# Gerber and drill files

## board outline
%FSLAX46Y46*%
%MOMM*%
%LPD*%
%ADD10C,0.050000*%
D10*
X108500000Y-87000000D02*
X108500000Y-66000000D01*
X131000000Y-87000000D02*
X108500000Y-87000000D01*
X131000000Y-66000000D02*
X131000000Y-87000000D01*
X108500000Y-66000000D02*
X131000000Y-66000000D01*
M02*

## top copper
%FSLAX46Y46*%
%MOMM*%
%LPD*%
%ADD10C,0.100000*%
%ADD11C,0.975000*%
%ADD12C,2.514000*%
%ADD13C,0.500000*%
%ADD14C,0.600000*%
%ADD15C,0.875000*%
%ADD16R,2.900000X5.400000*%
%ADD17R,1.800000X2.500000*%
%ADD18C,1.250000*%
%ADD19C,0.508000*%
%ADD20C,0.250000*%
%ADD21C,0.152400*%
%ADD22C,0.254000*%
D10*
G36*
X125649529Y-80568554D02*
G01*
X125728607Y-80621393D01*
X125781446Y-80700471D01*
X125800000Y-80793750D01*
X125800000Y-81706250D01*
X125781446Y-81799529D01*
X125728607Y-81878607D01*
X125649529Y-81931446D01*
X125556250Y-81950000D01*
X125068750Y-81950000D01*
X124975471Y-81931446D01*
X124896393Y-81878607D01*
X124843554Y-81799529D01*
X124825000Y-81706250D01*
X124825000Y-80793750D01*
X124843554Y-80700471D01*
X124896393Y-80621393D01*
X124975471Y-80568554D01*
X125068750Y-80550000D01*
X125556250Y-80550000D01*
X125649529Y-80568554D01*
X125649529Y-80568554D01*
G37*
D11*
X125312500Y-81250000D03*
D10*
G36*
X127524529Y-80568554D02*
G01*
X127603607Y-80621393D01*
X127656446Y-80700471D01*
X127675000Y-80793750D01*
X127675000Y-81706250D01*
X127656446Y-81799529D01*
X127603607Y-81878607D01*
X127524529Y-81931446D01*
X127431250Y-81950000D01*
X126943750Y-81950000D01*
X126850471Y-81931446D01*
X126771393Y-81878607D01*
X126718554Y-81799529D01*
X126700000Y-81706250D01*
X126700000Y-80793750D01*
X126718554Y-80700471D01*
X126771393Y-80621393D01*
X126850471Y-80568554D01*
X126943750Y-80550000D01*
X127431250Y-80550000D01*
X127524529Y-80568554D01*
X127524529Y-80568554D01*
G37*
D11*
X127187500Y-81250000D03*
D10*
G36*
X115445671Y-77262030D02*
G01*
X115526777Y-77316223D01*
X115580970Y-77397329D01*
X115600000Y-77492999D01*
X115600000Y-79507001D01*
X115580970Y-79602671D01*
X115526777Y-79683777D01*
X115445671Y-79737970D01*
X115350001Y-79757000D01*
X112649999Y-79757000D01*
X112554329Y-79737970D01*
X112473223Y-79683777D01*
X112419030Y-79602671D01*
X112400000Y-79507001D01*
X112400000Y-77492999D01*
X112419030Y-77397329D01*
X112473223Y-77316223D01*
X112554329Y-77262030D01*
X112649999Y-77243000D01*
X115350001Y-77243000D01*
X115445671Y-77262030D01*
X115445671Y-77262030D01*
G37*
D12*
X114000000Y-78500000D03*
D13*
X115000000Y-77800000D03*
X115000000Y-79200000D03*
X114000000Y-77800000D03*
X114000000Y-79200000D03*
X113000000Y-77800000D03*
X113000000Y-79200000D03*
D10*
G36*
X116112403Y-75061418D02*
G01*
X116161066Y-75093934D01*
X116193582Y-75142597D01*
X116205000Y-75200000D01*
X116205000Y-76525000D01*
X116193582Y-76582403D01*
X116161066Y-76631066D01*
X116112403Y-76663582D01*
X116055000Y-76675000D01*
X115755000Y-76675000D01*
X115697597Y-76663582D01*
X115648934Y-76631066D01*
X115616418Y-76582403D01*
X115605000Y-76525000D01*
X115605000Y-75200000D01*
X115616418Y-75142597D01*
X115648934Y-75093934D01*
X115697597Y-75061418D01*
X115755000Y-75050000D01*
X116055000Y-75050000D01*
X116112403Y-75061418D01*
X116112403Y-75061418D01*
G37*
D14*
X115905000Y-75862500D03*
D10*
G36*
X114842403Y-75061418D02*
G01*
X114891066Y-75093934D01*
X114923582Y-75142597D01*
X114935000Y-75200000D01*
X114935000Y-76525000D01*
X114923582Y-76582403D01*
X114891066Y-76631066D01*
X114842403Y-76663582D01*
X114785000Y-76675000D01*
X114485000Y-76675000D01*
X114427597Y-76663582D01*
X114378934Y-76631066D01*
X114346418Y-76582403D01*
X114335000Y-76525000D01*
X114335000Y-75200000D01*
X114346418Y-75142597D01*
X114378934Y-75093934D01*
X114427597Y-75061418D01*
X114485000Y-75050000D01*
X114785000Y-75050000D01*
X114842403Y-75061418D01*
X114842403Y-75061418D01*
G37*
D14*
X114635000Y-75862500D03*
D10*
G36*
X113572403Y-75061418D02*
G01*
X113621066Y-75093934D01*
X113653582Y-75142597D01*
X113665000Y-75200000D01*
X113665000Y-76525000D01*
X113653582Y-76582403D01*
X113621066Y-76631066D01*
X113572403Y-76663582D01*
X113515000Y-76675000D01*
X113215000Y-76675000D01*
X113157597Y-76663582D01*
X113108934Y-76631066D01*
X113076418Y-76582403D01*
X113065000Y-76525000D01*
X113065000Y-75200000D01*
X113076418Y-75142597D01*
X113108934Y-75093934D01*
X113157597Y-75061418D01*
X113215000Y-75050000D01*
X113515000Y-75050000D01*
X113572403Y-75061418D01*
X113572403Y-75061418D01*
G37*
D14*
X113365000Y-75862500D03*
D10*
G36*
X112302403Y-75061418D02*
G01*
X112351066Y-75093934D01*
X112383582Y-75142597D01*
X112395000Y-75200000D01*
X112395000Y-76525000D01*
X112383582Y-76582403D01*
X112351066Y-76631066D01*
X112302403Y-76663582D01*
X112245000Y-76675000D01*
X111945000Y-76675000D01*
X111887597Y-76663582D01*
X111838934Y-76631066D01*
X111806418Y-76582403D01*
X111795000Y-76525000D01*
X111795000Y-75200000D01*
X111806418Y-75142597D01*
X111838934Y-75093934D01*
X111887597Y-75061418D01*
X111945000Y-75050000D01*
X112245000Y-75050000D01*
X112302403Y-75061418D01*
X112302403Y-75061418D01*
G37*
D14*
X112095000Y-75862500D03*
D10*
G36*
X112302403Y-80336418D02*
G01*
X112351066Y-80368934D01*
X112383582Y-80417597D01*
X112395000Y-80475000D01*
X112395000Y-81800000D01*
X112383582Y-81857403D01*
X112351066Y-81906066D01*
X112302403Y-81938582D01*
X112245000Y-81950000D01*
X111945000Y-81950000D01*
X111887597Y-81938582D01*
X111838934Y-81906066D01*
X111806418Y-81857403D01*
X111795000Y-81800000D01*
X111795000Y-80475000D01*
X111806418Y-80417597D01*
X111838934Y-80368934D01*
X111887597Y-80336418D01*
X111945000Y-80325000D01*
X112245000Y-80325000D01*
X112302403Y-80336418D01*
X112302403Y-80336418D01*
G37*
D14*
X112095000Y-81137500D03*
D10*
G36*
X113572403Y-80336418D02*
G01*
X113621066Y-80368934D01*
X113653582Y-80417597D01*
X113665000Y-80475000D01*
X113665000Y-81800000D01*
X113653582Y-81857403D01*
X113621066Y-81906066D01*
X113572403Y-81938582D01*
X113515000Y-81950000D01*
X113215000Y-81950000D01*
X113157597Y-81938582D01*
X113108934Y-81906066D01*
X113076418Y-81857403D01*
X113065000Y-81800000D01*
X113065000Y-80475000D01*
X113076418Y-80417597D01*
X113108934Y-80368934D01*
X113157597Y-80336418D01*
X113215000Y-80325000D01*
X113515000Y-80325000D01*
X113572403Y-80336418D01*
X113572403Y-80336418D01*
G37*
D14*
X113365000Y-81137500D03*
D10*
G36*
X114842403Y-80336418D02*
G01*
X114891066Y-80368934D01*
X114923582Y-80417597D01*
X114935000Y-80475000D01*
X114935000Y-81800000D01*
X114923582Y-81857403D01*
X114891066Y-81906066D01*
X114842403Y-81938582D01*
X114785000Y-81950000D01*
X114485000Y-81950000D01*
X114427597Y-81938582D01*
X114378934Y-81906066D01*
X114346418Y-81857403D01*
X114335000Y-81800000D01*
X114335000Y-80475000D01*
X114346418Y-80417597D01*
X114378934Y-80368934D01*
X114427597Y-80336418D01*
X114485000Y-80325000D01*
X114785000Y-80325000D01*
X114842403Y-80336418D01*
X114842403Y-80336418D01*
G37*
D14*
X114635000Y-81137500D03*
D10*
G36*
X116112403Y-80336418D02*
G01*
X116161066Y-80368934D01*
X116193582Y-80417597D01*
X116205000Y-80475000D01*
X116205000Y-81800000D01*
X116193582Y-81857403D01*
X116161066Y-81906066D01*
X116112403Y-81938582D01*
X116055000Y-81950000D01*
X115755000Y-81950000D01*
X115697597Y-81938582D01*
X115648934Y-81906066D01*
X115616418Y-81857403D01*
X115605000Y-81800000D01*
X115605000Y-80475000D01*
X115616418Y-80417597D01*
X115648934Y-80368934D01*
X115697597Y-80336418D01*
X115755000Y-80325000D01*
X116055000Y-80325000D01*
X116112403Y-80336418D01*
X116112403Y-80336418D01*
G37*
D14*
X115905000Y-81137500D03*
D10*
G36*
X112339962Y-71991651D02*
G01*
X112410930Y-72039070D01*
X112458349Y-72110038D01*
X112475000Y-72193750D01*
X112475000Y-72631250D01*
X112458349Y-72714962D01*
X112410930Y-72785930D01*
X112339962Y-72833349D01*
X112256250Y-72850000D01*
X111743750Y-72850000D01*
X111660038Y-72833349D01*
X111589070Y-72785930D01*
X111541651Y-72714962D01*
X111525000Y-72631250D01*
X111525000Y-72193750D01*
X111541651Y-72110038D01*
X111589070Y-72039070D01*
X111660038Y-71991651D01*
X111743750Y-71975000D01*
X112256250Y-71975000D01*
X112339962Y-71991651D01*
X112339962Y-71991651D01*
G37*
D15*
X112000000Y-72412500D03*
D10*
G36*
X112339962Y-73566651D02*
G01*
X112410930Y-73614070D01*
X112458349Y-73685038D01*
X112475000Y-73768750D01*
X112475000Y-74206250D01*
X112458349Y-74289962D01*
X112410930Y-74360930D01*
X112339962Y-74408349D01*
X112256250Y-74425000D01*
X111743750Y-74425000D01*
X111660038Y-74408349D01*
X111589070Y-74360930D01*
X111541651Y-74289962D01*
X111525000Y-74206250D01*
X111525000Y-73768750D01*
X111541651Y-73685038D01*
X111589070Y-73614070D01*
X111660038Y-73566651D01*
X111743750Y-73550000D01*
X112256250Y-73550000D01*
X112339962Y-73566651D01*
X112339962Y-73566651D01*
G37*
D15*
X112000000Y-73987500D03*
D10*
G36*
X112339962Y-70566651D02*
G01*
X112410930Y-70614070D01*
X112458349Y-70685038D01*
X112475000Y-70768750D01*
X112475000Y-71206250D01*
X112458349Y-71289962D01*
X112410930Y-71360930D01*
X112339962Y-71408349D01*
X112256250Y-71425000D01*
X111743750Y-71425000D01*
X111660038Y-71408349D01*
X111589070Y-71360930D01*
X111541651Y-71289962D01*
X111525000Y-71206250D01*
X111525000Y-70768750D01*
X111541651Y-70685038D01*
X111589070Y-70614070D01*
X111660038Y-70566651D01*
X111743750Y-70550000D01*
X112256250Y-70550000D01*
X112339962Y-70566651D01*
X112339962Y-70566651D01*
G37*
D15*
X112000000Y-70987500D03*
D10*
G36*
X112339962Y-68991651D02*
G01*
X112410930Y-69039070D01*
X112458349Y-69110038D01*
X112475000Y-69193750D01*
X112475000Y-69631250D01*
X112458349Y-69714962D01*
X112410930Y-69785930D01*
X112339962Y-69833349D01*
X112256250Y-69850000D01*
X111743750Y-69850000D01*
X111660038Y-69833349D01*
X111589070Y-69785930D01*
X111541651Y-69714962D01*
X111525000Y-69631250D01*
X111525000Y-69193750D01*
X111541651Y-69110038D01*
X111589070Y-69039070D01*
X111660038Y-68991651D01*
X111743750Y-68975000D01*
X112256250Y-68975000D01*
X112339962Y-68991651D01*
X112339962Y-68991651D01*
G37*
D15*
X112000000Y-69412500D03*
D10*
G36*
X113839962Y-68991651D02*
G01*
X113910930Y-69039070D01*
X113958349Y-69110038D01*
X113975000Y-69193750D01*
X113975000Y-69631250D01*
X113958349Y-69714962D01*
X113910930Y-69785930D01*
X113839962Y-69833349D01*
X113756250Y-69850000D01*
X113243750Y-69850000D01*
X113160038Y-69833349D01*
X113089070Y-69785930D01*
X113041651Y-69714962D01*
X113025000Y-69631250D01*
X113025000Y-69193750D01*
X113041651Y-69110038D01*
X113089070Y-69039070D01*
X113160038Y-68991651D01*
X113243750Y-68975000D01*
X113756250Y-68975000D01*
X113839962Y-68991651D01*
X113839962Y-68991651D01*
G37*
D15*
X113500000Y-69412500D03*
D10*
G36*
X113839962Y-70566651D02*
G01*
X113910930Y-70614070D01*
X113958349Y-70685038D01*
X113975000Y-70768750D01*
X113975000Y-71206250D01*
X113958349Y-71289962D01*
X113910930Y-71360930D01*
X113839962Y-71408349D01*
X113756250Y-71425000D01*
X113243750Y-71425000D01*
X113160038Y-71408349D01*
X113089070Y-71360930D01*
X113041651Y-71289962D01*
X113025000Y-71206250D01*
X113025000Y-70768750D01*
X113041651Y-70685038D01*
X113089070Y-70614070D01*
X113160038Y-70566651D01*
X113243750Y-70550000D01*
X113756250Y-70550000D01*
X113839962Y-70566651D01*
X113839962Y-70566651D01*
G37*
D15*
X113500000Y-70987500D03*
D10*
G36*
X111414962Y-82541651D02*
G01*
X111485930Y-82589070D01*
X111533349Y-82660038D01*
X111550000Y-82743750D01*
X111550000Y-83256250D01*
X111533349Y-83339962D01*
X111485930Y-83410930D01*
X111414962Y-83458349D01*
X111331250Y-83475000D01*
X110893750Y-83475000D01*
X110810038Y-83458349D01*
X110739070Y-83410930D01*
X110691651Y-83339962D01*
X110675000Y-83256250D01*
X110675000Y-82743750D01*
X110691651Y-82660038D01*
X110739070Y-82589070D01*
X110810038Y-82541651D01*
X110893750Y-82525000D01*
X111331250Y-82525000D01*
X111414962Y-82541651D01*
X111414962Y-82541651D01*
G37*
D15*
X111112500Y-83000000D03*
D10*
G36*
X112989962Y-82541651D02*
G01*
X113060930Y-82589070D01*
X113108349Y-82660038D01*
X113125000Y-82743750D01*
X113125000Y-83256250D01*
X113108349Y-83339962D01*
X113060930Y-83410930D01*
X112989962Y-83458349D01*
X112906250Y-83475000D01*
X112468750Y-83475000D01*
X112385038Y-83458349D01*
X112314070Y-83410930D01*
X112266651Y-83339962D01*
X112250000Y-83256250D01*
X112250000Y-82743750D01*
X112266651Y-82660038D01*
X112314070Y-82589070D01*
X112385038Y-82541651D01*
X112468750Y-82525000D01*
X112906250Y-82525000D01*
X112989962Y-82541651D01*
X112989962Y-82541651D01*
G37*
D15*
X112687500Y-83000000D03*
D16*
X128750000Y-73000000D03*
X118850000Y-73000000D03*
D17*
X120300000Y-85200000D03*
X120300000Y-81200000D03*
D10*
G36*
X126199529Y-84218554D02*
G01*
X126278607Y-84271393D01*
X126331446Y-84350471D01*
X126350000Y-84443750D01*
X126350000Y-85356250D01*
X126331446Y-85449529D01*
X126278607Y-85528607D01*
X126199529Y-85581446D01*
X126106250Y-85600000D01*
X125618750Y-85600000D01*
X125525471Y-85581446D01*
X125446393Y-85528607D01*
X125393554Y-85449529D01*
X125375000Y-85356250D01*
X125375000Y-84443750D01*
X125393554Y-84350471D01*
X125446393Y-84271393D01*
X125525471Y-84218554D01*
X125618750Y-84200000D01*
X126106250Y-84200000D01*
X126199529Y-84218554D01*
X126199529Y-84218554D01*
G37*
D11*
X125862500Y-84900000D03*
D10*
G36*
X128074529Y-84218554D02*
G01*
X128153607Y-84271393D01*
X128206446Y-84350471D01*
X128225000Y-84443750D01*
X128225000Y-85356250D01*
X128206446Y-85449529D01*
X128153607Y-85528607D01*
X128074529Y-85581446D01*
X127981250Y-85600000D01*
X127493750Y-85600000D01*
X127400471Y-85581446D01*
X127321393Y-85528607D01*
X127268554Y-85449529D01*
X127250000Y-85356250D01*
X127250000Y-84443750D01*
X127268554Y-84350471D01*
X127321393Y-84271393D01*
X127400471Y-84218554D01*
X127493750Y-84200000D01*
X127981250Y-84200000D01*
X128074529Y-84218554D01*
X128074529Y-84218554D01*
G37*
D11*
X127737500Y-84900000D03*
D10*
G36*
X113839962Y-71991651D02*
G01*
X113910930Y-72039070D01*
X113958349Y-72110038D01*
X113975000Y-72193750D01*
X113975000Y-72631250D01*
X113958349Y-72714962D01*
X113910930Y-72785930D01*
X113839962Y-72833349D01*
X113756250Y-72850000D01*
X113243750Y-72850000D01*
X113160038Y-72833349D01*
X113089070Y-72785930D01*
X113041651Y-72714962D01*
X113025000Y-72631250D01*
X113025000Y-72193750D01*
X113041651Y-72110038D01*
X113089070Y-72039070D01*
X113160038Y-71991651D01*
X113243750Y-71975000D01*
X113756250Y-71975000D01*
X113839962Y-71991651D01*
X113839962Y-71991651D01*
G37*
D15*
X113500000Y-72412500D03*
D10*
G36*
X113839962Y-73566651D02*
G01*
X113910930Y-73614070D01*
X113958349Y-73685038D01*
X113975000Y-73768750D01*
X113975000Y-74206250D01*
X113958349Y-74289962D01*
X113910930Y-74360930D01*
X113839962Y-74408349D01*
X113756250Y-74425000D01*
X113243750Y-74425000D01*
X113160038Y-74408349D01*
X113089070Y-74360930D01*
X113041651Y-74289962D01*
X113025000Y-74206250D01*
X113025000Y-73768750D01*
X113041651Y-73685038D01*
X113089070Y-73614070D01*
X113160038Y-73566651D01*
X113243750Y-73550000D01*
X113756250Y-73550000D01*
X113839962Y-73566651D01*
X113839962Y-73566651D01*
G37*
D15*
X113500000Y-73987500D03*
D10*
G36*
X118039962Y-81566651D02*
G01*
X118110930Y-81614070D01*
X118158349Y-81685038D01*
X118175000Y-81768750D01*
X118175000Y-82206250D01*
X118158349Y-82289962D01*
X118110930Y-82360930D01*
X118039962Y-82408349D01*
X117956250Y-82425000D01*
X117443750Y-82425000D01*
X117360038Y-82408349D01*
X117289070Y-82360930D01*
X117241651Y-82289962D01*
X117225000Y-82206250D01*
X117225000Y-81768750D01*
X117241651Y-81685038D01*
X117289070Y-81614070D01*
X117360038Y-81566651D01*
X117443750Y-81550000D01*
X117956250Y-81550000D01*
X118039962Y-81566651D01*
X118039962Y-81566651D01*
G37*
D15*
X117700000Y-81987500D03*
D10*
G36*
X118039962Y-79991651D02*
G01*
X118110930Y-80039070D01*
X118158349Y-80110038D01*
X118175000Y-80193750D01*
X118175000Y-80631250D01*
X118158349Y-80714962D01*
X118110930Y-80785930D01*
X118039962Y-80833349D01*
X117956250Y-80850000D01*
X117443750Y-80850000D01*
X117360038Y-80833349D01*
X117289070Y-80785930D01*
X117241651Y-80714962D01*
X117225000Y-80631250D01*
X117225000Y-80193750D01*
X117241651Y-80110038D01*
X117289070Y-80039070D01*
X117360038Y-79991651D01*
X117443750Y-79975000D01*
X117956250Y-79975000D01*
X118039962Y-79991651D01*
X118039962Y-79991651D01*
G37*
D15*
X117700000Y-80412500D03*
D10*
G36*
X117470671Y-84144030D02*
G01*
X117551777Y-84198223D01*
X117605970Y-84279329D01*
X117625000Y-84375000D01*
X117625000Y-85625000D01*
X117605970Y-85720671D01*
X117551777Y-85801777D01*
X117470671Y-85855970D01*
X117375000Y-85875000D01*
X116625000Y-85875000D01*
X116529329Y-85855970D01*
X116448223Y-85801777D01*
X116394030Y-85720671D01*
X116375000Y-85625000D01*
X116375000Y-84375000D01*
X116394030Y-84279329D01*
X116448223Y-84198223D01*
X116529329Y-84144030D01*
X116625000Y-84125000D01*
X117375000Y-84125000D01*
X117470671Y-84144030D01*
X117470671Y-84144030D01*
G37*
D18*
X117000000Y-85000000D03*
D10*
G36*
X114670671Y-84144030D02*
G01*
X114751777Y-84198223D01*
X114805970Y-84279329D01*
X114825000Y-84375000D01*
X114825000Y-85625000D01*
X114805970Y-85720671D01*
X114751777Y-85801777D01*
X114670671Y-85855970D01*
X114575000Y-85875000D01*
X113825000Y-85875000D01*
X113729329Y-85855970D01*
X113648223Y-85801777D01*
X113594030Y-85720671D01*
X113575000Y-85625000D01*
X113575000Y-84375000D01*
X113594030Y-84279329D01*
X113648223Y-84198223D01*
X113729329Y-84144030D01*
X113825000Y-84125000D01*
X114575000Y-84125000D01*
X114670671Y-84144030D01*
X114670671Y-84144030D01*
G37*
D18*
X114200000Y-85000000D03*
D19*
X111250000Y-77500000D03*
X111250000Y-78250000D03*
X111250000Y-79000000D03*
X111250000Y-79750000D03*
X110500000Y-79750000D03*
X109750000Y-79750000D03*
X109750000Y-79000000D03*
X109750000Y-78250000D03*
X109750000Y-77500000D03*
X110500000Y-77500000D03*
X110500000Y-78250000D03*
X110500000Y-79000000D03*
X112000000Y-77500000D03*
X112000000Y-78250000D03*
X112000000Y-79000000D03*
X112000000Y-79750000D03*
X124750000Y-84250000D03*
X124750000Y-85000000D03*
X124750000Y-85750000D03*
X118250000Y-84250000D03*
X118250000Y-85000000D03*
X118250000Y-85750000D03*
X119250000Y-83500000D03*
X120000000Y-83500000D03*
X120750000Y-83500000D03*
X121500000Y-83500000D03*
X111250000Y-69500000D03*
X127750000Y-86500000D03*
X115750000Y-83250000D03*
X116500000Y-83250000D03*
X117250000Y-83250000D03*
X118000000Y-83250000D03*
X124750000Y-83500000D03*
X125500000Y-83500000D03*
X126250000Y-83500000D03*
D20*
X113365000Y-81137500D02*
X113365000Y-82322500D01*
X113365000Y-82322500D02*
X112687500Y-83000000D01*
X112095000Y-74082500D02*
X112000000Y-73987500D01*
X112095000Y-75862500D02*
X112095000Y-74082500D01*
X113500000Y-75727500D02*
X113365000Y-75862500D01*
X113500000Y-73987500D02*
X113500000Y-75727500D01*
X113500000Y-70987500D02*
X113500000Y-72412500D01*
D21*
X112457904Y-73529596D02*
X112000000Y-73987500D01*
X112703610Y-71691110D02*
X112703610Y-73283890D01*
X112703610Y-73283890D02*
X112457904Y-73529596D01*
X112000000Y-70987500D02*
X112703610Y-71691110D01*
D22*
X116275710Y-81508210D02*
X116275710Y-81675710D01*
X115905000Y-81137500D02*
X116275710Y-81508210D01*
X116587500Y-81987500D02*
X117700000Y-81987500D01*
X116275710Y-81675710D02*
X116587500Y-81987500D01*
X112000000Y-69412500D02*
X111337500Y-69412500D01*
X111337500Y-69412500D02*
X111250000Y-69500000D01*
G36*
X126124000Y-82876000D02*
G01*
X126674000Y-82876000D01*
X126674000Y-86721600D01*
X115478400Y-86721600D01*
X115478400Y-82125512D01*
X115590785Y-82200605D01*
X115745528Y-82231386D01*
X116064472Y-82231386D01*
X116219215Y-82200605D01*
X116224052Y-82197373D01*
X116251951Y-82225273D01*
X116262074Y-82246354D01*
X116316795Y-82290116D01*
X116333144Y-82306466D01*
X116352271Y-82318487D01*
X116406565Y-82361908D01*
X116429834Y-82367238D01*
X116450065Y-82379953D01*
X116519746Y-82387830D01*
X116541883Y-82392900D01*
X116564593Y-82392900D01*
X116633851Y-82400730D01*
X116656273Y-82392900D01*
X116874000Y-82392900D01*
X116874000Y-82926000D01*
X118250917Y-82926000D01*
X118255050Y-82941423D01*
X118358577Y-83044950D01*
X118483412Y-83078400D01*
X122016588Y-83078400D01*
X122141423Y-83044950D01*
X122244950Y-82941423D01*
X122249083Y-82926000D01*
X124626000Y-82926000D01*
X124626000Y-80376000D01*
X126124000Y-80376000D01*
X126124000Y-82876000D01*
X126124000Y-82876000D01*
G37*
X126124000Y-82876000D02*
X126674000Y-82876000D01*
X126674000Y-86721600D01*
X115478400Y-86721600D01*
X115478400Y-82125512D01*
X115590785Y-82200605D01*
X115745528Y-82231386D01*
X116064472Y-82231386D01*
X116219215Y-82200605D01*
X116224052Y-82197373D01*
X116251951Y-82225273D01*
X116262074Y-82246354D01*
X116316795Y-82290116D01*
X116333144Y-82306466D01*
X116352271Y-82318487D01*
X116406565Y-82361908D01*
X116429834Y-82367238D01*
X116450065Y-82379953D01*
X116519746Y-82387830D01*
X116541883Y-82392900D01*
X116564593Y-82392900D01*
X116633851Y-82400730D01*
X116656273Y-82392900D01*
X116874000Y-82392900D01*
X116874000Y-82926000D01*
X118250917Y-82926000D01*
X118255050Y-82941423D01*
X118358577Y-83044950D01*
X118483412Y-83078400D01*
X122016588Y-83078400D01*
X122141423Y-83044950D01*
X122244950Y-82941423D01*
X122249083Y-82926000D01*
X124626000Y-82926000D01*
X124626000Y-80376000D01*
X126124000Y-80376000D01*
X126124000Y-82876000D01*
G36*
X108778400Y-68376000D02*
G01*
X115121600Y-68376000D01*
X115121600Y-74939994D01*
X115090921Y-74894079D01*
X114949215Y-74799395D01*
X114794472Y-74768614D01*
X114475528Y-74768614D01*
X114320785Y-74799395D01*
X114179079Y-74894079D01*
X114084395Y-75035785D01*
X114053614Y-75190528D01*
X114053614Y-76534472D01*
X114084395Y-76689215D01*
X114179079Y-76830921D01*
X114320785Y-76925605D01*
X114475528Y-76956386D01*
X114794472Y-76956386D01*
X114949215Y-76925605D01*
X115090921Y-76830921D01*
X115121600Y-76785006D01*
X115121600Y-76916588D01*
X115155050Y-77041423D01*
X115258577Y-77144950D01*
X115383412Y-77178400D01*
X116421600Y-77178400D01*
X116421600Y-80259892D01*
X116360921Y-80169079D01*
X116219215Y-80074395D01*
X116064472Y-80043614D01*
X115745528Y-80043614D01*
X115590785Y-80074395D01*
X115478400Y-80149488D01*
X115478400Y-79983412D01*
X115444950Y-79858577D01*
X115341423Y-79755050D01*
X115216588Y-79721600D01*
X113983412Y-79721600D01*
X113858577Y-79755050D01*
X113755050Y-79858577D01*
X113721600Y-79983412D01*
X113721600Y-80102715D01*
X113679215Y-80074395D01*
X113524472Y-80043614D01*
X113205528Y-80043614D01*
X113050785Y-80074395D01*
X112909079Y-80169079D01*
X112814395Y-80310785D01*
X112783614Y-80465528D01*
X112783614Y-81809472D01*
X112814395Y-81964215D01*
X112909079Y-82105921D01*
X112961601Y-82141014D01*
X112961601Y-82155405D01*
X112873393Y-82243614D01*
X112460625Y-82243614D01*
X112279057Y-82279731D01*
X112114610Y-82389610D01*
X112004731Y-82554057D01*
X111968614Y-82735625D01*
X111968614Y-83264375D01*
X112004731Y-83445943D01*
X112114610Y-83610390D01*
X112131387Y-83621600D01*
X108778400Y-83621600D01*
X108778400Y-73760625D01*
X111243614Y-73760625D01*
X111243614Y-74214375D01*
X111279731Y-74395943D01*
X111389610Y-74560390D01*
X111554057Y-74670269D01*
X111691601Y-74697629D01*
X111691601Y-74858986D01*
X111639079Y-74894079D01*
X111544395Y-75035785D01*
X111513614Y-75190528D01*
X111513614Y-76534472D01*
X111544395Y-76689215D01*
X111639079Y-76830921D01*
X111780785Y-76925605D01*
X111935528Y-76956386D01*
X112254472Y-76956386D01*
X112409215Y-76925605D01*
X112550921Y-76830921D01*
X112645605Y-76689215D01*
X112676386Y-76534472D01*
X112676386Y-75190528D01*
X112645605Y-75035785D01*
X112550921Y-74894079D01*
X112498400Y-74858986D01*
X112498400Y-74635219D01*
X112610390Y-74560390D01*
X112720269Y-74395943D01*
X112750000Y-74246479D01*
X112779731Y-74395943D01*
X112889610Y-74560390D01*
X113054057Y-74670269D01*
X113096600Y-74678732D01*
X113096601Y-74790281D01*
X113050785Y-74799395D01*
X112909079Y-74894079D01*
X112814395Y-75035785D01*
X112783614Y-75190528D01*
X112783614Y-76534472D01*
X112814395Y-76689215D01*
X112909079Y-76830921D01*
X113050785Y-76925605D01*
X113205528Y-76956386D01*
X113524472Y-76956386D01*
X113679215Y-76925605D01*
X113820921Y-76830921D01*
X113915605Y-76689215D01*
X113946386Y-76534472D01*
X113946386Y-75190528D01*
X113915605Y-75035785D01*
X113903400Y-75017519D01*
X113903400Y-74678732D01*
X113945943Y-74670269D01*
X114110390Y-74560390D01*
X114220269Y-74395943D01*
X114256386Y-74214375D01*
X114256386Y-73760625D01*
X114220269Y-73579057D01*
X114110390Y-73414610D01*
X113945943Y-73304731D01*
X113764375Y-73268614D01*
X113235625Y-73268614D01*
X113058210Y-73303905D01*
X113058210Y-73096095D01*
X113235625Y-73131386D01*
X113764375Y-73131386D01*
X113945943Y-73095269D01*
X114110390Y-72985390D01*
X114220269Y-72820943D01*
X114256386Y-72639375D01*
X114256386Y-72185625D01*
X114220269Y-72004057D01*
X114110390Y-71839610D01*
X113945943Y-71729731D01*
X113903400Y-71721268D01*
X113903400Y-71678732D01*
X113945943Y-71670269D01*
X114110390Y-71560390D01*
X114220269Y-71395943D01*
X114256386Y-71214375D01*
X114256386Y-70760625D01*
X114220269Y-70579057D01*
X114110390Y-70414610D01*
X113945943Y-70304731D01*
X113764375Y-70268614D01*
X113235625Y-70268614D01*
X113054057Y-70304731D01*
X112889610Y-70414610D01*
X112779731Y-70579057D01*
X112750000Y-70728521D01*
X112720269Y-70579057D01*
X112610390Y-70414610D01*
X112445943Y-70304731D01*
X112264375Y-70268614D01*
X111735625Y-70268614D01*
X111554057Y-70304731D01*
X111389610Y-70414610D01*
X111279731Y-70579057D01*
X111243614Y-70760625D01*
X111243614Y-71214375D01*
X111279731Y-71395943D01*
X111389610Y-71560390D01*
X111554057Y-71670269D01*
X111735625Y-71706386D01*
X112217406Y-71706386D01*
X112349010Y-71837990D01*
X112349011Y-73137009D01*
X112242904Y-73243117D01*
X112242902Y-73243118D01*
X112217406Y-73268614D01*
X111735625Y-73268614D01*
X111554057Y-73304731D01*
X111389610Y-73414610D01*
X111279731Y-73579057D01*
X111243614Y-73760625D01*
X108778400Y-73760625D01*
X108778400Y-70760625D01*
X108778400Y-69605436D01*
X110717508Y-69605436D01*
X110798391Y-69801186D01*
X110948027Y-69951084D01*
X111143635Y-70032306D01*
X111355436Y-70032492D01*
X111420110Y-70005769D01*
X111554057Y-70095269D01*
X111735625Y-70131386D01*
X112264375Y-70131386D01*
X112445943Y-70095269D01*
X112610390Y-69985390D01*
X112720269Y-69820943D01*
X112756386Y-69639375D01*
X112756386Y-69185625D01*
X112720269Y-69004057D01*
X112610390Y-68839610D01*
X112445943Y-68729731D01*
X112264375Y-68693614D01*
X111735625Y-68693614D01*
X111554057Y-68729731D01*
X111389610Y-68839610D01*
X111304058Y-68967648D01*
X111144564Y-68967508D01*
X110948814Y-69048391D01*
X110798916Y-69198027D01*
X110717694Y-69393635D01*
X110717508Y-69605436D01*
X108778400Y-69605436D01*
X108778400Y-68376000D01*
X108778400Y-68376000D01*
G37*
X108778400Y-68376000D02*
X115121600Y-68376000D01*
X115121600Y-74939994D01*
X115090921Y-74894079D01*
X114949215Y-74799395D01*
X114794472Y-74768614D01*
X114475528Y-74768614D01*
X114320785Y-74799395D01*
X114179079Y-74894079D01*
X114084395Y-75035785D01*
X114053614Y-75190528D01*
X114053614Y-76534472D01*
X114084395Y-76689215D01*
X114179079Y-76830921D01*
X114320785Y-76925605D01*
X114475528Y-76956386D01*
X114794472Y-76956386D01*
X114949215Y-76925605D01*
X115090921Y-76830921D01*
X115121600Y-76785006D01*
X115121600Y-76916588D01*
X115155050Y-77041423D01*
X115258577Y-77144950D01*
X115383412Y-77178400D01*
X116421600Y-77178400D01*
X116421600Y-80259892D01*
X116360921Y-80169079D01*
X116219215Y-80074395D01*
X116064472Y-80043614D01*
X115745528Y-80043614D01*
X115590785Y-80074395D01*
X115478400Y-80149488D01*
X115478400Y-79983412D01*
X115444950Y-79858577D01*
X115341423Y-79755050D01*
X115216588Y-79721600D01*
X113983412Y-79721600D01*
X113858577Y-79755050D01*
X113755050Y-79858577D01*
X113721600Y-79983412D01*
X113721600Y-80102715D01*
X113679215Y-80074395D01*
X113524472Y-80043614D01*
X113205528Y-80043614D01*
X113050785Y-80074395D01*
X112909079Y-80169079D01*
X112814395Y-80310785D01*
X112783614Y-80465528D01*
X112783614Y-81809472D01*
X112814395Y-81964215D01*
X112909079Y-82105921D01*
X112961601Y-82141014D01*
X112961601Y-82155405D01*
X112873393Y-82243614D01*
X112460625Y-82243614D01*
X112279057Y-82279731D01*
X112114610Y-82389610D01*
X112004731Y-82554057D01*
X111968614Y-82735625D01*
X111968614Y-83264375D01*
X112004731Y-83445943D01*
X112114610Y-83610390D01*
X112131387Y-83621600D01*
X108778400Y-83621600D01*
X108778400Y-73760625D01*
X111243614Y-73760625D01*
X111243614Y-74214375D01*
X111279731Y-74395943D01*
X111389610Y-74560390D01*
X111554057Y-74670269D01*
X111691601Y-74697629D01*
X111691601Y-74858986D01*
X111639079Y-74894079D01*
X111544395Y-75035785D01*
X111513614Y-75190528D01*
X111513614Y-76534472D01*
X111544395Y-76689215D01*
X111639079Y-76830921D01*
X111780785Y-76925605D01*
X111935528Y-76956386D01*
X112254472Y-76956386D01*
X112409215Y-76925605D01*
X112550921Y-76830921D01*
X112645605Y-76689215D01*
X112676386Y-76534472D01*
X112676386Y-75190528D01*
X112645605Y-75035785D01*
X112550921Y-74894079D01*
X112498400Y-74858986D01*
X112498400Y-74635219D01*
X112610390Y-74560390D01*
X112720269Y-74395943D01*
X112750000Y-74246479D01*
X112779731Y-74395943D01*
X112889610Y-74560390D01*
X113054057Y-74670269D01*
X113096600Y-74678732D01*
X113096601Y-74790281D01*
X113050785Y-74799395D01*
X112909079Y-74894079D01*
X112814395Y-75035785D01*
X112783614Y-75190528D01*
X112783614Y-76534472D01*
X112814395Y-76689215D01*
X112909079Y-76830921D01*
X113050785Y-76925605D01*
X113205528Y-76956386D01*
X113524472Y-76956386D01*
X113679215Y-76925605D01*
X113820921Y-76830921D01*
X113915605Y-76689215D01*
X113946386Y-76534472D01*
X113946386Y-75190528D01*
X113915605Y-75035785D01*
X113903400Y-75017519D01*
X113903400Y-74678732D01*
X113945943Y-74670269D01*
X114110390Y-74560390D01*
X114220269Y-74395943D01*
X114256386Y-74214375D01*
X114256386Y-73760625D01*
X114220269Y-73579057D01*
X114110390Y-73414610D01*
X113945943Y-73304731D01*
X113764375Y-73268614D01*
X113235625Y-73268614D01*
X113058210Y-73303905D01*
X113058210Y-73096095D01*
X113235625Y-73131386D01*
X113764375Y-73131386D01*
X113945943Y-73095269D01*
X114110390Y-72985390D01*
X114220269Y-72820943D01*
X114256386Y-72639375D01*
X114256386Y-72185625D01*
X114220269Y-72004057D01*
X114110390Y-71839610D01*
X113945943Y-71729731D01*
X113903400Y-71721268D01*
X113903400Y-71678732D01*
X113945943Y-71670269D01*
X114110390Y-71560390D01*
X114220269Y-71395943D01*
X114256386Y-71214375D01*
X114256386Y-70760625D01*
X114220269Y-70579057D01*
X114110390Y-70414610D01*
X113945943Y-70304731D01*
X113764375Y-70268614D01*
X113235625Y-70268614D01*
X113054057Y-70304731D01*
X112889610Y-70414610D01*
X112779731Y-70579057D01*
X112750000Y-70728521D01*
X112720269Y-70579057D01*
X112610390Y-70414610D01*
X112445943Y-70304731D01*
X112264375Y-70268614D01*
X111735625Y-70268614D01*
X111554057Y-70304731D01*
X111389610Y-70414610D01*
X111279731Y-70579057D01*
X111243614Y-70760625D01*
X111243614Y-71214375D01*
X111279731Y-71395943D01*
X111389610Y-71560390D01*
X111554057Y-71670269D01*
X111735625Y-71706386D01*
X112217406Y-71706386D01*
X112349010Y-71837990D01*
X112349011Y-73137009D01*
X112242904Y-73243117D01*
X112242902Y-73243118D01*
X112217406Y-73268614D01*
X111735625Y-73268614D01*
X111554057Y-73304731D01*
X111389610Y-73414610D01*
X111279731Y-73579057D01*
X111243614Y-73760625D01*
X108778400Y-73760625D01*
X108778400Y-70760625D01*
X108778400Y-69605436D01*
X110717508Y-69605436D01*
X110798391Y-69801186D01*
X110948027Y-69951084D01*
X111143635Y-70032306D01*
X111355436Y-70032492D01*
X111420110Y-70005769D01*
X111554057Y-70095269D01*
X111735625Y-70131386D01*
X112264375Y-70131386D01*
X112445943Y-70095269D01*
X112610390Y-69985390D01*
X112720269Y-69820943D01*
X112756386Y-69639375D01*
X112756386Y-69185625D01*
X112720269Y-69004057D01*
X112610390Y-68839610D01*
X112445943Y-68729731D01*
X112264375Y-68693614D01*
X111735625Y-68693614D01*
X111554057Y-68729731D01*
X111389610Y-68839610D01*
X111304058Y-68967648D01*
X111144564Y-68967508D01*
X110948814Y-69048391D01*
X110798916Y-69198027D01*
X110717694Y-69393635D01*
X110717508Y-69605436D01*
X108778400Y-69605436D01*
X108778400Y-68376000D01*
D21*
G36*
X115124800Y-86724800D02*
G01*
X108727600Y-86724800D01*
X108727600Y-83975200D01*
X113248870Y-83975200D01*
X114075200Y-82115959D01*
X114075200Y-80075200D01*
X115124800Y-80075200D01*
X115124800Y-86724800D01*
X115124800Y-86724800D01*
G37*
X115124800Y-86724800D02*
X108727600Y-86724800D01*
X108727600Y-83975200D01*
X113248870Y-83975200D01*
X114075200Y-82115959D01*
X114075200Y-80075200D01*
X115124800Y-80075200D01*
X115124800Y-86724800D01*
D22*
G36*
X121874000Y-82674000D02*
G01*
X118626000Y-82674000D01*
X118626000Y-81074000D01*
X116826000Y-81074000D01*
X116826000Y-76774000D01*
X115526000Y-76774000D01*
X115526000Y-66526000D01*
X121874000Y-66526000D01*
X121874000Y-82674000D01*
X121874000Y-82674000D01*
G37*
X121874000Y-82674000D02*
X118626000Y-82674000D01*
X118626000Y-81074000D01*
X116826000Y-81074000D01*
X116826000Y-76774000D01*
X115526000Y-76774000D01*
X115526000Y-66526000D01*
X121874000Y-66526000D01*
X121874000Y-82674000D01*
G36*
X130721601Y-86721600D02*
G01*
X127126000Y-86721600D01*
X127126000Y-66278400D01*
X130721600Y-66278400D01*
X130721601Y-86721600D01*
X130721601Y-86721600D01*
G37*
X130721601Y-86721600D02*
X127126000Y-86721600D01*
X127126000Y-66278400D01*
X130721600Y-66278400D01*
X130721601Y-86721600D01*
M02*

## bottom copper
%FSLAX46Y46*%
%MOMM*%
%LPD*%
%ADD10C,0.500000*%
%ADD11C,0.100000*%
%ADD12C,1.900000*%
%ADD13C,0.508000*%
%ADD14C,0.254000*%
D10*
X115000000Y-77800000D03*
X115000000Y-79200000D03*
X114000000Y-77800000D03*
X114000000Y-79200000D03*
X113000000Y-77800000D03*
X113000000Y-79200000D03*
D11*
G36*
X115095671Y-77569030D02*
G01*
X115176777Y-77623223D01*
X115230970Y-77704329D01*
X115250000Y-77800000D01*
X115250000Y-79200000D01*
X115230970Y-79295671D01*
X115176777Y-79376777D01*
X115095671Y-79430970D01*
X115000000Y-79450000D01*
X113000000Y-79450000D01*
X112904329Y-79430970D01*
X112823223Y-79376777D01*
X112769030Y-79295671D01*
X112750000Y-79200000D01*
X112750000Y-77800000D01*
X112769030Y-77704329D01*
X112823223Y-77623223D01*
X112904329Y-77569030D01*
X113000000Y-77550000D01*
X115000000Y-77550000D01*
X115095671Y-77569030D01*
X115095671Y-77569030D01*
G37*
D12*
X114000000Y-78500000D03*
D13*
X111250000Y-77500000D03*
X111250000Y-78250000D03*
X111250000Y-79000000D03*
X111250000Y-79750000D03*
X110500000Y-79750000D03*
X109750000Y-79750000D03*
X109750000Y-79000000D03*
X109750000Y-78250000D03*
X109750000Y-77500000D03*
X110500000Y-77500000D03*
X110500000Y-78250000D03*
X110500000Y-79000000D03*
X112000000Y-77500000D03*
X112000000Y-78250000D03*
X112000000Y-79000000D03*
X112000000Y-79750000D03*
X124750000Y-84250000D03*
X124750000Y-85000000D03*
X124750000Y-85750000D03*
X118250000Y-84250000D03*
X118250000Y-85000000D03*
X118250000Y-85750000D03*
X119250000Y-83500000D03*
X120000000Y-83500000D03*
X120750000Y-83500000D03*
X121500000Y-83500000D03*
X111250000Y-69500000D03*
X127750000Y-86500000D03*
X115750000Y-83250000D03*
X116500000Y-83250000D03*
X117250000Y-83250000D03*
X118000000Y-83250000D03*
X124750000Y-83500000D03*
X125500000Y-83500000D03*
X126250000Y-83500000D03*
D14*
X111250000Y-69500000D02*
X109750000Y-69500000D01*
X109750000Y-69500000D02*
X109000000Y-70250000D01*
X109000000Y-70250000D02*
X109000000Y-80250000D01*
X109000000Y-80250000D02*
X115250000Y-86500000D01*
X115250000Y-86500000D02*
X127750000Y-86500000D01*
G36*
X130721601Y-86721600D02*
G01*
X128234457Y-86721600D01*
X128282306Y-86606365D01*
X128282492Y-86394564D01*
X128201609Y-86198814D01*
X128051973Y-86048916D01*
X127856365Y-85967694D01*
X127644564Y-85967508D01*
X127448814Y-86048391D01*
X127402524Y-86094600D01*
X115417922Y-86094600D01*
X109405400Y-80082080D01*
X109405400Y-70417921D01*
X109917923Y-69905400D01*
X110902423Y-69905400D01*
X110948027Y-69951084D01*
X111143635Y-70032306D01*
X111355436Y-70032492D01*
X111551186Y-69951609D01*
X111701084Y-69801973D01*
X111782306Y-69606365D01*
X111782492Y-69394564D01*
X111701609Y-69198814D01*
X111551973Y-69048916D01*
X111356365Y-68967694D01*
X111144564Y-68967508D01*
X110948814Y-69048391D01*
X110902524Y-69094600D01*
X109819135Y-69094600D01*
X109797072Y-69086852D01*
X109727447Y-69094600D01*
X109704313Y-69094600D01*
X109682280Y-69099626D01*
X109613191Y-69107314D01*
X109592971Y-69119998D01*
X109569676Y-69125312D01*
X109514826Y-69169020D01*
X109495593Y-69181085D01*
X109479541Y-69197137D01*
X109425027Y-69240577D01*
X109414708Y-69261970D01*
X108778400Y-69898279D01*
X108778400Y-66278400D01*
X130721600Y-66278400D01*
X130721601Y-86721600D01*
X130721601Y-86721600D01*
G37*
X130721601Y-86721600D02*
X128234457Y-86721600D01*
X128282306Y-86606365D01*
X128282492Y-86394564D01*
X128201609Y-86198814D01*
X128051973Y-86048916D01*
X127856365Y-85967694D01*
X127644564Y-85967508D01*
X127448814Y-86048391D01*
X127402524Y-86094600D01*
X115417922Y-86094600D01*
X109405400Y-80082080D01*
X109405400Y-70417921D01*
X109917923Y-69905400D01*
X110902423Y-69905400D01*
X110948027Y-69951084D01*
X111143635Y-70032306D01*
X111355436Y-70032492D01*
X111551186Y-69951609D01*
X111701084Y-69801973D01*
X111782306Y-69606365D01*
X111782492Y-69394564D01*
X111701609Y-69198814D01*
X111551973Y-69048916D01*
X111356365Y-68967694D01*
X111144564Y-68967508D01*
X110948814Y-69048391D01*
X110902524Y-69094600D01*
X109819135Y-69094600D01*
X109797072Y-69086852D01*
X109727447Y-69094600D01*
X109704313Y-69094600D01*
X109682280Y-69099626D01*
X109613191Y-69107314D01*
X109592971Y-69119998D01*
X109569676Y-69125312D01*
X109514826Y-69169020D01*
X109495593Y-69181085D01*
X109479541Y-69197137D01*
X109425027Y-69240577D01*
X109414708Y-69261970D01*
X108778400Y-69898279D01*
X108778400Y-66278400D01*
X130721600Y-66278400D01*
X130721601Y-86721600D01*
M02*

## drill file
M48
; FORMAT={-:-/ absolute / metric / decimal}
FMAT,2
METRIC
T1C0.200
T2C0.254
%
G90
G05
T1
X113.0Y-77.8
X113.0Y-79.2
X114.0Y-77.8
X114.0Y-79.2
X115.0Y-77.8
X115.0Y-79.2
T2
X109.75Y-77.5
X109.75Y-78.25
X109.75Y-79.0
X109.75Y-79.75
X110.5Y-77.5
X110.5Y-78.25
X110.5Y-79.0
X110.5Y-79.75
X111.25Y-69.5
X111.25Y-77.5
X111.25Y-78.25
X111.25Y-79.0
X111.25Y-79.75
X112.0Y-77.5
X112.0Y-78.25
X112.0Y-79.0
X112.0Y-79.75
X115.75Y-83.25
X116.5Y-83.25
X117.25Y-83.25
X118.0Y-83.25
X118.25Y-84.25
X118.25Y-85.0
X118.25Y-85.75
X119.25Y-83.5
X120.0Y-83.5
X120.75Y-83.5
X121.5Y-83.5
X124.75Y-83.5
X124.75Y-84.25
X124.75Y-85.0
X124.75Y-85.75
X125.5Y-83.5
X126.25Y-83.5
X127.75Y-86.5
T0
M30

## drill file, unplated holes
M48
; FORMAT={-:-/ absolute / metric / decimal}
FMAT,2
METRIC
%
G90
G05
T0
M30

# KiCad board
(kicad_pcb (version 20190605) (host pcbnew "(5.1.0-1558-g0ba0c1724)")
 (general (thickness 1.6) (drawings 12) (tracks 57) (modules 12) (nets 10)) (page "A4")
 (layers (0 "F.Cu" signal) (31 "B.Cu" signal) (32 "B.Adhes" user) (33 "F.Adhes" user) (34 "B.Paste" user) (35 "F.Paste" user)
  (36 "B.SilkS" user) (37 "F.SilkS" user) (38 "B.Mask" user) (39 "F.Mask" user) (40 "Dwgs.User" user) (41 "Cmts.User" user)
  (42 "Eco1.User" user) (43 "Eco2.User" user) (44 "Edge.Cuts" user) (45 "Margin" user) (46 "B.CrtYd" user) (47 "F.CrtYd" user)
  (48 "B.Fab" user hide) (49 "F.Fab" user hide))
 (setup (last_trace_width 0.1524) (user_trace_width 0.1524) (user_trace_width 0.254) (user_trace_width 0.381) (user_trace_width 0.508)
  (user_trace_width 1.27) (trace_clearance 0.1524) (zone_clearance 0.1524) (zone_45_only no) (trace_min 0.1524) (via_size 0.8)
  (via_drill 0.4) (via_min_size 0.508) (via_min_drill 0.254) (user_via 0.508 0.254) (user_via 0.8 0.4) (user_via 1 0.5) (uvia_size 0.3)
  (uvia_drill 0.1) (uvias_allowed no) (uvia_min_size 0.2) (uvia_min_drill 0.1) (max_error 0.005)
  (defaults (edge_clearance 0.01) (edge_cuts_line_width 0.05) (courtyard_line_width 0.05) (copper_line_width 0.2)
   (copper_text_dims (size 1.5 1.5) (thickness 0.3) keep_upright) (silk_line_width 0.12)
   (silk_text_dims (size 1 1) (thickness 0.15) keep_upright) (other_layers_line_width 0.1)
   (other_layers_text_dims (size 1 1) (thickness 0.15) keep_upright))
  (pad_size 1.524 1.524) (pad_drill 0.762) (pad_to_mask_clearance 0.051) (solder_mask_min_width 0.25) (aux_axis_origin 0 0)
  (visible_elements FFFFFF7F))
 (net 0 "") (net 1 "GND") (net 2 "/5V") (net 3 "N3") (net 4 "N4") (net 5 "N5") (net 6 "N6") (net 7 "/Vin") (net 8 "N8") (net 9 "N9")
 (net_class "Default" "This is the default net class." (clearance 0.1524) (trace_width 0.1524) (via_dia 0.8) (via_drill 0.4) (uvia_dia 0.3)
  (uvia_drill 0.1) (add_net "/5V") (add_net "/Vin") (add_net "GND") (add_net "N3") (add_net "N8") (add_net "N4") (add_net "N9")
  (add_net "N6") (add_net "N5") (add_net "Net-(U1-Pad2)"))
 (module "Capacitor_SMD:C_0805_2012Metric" (layer "F.Cu") (at 126.25 81.25 180)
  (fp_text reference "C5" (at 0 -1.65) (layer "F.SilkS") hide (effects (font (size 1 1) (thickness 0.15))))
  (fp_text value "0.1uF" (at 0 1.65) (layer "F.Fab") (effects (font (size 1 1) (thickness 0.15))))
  (pad "2" smd roundrect (at 0.9375 0 180) (size 0.975 1.4) (layers "F.Cu" "F.Paste" "F.Mask") (roundrect_rratio 0.25) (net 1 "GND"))
  (pad "1" smd roundrect (at -0.9375 0 180) (size 0.975 1.4) (layers "F.Cu" "F.Paste" "F.Mask") (roundrect_rratio 0.25) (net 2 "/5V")))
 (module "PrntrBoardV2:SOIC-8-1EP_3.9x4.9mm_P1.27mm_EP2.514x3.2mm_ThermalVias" (layer "F.Cu") (at 114 78.5 270)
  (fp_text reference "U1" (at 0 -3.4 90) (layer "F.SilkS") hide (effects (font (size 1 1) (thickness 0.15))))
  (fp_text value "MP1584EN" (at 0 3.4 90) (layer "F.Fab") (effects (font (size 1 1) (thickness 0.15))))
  (pad "9" smd roundrect (at 0 0 270) (size 2.514 3.2) (layers "F.Cu" "F.Mask") (roundrect_rratio 0.099443) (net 1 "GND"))
  (pad "9" thru_hole circle (at -0.7 -1 270) (size 0.5 0.5) (drill 0.2) (layers *.Cu) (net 1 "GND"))
  (pad "9" thru_hole circle (at 0.7 -1 270) (size 0.5 0.5) (drill 0.2) (layers *.Cu) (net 1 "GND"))
  (pad "9" thru_hole circle (at -0.7 0 270) (size 0.5 0.5) (drill 0.2) (layers *.Cu) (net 1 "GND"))
  (pad "9" thru_hole circle (at 0.7 0 270) (size 0.5 0.5) (drill 0.2) (layers *.Cu) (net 1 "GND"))
  (pad "9" thru_hole circle (at -0.7 1 270) (size 0.5 0.5) (drill 0.2) (layers *.Cu) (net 1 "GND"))
  (pad "9" thru_hole circle (at 0.7 1 270) (size 0.5 0.5) (drill 0.2) (layers *.Cu) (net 1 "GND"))
  (pad "9" smd roundrect (at 0 0 270) (size 1.9 2.5) (layers "B.Cu") (roundrect_rratio 0.131579) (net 1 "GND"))
  (pad "" smd roundrect (at -0.63 -0.8 270) (size 1.05 1.34) (layers "F.Paste") (roundrect_rratio 0.238095))
  (pad "" smd roundrect (at -0.63 0.8 270) (size 1.05 1.34) (layers "F.Paste") (roundrect_rratio 0.238095))
  (pad "" smd roundrect (at 0.63 -0.8 270) (size 1.05 1.34) (layers "F.Paste") (roundrect_rratio 0.238095))
  (pad "" smd roundrect (at 0.63 0.8 270) (size 1.05 1.34) (layers "F.Paste") (roundrect_rratio 0.238095))
  (pad "1" smd roundrect (at -2.6375 -1.905 270) (size 1.625 0.6) (layers "F.Cu" "F.Paste" "F.Mask") (roundrect_rratio 0.25) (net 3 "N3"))
  (pad "2" smd roundrect (at -2.6375 -0.635 270) (size 1.625 0.6) (layers "F.Cu" "F.Paste" "F.Mask") (roundrect_rratio 0.25))
  (pad "3" smd roundrect (at -2.6375 0.635 270) (size 1.625 0.6) (layers "F.Cu" "F.Paste" "F.Mask") (roundrect_rratio 0.25) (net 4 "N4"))
  (pad "4" smd roundrect (at -2.6375 1.905 270) (size 1.625 0.6) (layers "F.Cu" "F.Paste" "F.Mask") (roundrect_rratio 0.25) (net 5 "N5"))
  (pad "5" smd roundrect (at 2.6375 1.905 270) (size 1.625 0.6) (layers "F.Cu" "F.Paste" "F.Mask") (roundrect_rratio 0.25) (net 1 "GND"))
  (pad "6" smd roundrect (at 2.6375 0.635 270) (size 1.625 0.6) (layers "F.Cu" "F.Paste" "F.Mask") (roundrect_rratio 0.25) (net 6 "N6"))
  (pad "7" smd roundrect (at 2.6375 -0.635 270) (size 1.625 0.6) (layers "F.Cu" "F.Paste" "F.Mask") (roundrect_rratio 0.25) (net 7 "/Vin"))
  (pad "8" smd roundrect (at 2.6375 -1.905 270) (size 1.625 0.6) (layers "F.Cu" "F.Paste" "F.Mask") (roundrect_rratio 0.25) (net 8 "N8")))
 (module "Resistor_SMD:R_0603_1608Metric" (layer "F.Cu") (at 112 73.2 90)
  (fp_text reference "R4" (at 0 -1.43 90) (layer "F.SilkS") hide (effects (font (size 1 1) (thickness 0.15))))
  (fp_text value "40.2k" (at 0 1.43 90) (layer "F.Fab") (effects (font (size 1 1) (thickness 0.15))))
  (pad "2" smd roundrect (at 0.7875 0 90) (size 0.875 0.95) (layers "F.Cu" "F.Paste" "F.Mask") (roundrect_rratio 0.25) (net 1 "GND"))
  (pad "1" smd roundrect (at -0.7875 0 90) (size 0.875 0.95) (layers "F.Cu" "F.Paste" "F.Mask") (roundrect_rratio 0.25) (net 5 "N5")))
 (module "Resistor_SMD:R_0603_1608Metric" (layer "F.Cu") (at 112 70.2 270)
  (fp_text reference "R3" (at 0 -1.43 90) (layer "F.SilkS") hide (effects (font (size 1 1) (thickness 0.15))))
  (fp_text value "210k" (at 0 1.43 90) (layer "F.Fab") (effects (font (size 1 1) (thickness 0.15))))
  (pad "2" smd roundrect (at 0.7875 0 270) (size 0.875 0.95) (layers "F.Cu" "F.Paste" "F.Mask") (roundrect_rratio 0.25) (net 5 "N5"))
  (pad "1" smd roundrect (at -0.7875 0 270) (size 0.875 0.95) (layers "F.Cu" "F.Paste" "F.Mask") (roundrect_rratio 0.25) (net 2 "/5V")))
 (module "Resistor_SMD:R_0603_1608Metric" (layer "F.Cu") (at 113.5 70.2 90)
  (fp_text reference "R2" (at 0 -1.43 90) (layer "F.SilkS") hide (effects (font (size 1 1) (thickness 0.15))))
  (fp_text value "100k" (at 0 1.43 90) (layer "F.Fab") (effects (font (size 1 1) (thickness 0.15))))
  (pad "2" smd roundrect (at 0.7875 0 90) (size 0.875 0.95) (layers "F.Cu" "F.Paste" "F.Mask") (roundrect_rratio 0.25) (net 1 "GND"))
  (pad "1" smd roundrect (at -0.7875 0 90) (size 0.875 0.95) (layers "F.Cu" "F.Paste" "F.Mask") (roundrect_rratio 0.25) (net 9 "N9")))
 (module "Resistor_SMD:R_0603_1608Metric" (layer "F.Cu") (at 111.9 83 180)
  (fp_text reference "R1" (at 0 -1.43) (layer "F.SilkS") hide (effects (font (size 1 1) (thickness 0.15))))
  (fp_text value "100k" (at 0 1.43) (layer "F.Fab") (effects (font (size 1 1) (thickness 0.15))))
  (pad "2" smd roundrect (at 0.7875 0 180) (size 0.875 0.95) (layers "F.Cu" "F.Paste" "F.Mask") (roundrect_rratio 0.25) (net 1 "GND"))
  (pad "1" smd roundrect (at -0.7875 0 180) (size 0.875 0.95) (layers "F.Cu" "F.Paste" "F.Mask") (roundrect_rratio 0.25) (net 6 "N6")))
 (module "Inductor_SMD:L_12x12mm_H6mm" (layer "F.Cu") (at 123.8 73)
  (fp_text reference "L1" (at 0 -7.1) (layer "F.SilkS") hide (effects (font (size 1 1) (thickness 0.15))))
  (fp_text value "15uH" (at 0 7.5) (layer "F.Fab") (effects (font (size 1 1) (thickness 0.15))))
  (pad "2" smd rect (at 4.95 0) (size 2.9 5.4) (layers "F.Cu" "F.Paste" "F.Mask") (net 2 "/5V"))
  (pad "1" smd rect (at -4.95 0) (size 2.9 5.4) (layers "F.Cu" "F.Paste" "F.Mask") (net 3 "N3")))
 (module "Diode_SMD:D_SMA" (layer "F.Cu") (at 120.3 83.2 270)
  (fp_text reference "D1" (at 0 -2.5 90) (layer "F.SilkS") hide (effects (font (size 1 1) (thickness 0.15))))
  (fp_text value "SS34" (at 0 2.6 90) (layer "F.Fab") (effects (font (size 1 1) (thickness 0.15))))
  (pad "2" smd rect (at 2 0 270) (size 2.5 1.8) (layers "F.Cu" "F.Paste" "F.Mask") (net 1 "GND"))
  (pad "1" smd rect (at -2 0 270) (size 2.5 1.8) (layers "F.Cu" "F.Paste" "F.Mask") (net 3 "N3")))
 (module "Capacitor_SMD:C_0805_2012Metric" (layer "F.Cu") (at 126.8 84.9 180)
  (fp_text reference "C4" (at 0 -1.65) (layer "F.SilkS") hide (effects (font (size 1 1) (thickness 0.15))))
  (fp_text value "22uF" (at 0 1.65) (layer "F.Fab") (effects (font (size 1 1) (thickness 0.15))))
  (pad "2" smd roundrect (at 0.9375 0 180) (size 0.975 1.4) (layers "F.Cu" "F.Paste" "F.Mask") (roundrect_rratio 0.25) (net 1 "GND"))
  (pad "1" smd roundrect (at -0.9375 0 180) (size 0.975 1.4) (layers "F.Cu" "F.Paste" "F.Mask") (roundrect_rratio 0.25) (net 2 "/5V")))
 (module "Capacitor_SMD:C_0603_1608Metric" (layer "F.Cu") (at 113.5 73.2 90)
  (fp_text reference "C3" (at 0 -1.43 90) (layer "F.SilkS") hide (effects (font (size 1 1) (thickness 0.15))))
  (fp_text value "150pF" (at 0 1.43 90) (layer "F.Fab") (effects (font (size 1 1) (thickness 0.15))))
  (pad "2" smd roundrect (at 0.7875 0 90) (size 0.875 0.95) (layers "F.Cu" "F.Paste" "F.Mask") (roundrect_rratio 0.25) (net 9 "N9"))
  (pad "1" smd roundrect (at -0.7875 0 90) (size 0.875 0.95) (layers "F.Cu" "F.Paste" "F.Mask") (roundrect_rratio 0.25) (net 4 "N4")))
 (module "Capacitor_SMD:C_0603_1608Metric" (layer "F.Cu") (at 117.7 81.2 270)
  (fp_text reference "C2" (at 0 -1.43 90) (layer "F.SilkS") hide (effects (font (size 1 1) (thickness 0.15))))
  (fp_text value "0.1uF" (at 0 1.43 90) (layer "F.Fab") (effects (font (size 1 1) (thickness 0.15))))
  (pad "2" smd roundrect (at 0.7875 0 270) (size 0.875 0.95) (layers "F.Cu" "F.Paste" "F.Mask") (roundrect_rratio 0.25) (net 8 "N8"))
  (pad "1" smd roundrect (at -0.7875 0 270) (size 0.875 0.95) (layers "F.Cu" "F.Paste" "F.Mask") (roundrect_rratio 0.25) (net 3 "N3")))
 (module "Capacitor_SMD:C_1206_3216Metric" (layer "F.Cu") (at 115.6 85)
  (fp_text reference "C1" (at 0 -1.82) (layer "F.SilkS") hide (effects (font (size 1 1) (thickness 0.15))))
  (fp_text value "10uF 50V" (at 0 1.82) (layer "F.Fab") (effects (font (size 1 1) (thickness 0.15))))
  (pad "2" smd roundrect (at 1.4 0) (size 1.25 1.75) (layers "F.Cu" "F.Paste" "F.Mask") (roundrect_rratio 0.2) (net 1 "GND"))
  (pad "1" smd roundrect (at -1.4 0) (size 1.25 1.75) (layers "F.Cu" "F.Paste" "F.Mask") (roundrect_rratio 0.2) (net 7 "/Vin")))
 (gr_line (start 108.5 87) (end 108.5 66) (layer "Edge.Cuts") (width 0.05))
 (gr_line (start 131 87) (end 108.5 87) (layer "Edge.Cuts") (width 0.05))
 (gr_line (start 131 66) (end 131 87) (layer "Edge.Cuts") (width 0.05))
 (gr_line (start 108.5 66) (end 131 66) (layer "Edge.Cuts") (width 0.05))
 (segment (start 113.365 81.1375) (end 113.365 82.3225) (width 0.25) (layer "F.Cu") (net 6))
 (segment (start 113.365 82.3225) (end 112.6875 83) (width 0.25) (layer "F.Cu") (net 6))
 (segment (start 112.095 74.0825) (end 112 73.9875) (width 0.25) (layer "F.Cu") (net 5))
 (segment (start 112.095 75.8625) (end 112.095 74.0825) (width 0.25) (layer "F.Cu") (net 5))
 (segment (start 113.5 75.7275) (end 113.365 75.8625) (width 0.25) (layer "F.Cu") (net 4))
 (segment (start 113.5 73.9875) (end 113.5 75.7275) (width 0.25) (layer "F.Cu") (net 4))
 (segment (start 113.5 70.9875) (end 113.5 72.4125) (width 0.25) (layer "F.Cu") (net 9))
 (segment (start 112.457904 73.529596) (end 112 73.9875) (width 0.1524) (layer "F.Cu") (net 5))
 (segment (start 112.70361 71.69111) (end 112.70361 73.28389) (width 0.1524) (layer "F.Cu") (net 5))
 (segment (start 112.70361 73.28389) (end 112.457904 73.529596) (width 0.1524) (layer "F.Cu") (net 5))
 (segment (start 112 70.9875) (end 112.70361 71.69111) (width 0.1524) (layer "F.Cu") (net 5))
 (segment (start 116.27571 81.50821) (end 116.27571 81.67571) (width 0.254) (layer "F.Cu") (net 8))
 (segment (start 115.905 81.1375) (end 116.27571 81.50821) (width 0.254) (layer "F.Cu") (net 8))
 (segment (start 116.5875 81.9875) (end 117.7 81.9875) (width 0.254) (layer "F.Cu") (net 8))
 (segment (start 116.27571 81.67571) (end 116.5875 81.9875) (width 0.254) (layer "F.Cu") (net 8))
 (via (at 111.25 77.5) (size 0.508) (drill 0.254) (layers "F.Cu" "B.Cu") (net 1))
 (via (at 111.25 78.25) (size 0.508) (drill 0.254) (layers "F.Cu" "B.Cu") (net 1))
 (via (at 111.25 79) (size 0.508) (drill 0.254) (layers "F.Cu" "B.Cu") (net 1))
 (via (at 111.25 79.75) (size 0.508) (drill 0.254) (layers "F.Cu" "B.Cu") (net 1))
 (via (at 110.5 79.75) (size 0.508) (drill 0.254) (layers "F.Cu" "B.Cu") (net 1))
 (via (at 109.75 79.75) (size 0.508) (drill 0.254) (layers "F.Cu" "B.Cu") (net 1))
 (via (at 109.75 79) (size 0.508) (drill 0.254) (layers "F.Cu" "B.Cu") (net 1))
 (via (at 109.75 78.25) (size 0.508) (drill 0.254) (layers "F.Cu" "B.Cu") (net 1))
 (via (at 109.75 77.5) (size 0.508) (drill 0.254) (layers "F.Cu" "B.Cu") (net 1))
 (via (at 110.5 77.5) (size 0.508) (drill 0.254) (layers "F.Cu" "B.Cu") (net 1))
 (via (at 110.5 78.25) (size 0.508) (drill 0.254) (layers "F.Cu" "B.Cu") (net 1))
 (via (at 110.5 79) (size 0.508) (drill 0.254) (layers "F.Cu" "B.Cu") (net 1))
 (via (at 112 77.5) (size 0.508) (drill 0.254) (layers "F.Cu" "B.Cu") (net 1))
 (via (at 112 78.25) (size 0.508) (drill 0.254) (layers "F.Cu" "B.Cu") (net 1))
 (via (at 112 79) (size 0.508) (drill 0.254) (layers "F.Cu" "B.Cu") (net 1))
 (via (at 112 79.75) (size 0.508) (drill 0.254) (layers "F.Cu" "B.Cu") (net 1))
 (via (at 124.75 84.25) (size 0.508) (drill 0.254) (layers "F.Cu" "B.Cu") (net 1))
 (via (at 124.75 85) (size 0.508) (drill 0.254) (layers "F.Cu" "B.Cu") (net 1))
 (via (at 124.75 85.75) (size 0.508) (drill 0.254) (layers "F.Cu" "B.Cu") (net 1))
 (via (at 118.25 84.25) (size 0.508) (drill 0.254) (layers "F.Cu" "B.Cu") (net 1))
 (via (at 118.25 85) (size 0.508) (drill 0.254) (layers "F.Cu" "B.Cu") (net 1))
 (via (at 118.25 85.75) (size 0.508) (drill 0.254) (layers "F.Cu" "B.Cu") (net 1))
 (via (at 119.25 83.5) (size 0.508) (drill 0.254) (layers "F.Cu" "B.Cu") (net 1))
 (via (at 120 83.5) (size 0.508) (drill 0.254) (layers "F.Cu" "B.Cu") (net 1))
 (via (at 120.75 83.5) (size 0.508) (drill 0.254) (layers "F.Cu" "B.Cu") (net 1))
 (via (at 121.5 83.5) (size 0.508) (drill 0.254) (layers "F.Cu" "B.Cu") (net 1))
 (via (at 111.25 69.5) (size 0.508) (drill 0.254) (layers "F.Cu" "B.Cu") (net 2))
 (segment (start 112 69.4125) (end 111.3375 69.4125) (width 0.254) (layer "F.Cu") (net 2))
 (segment (start 111.3375 69.4125) (end 111.25 69.5) (width 0.254) (layer "F.Cu") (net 2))
 (segment (start 111.25 69.5) (end 109.75 69.5) (width 0.254) (layer "B.Cu") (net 2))
 (segment (start 109.75 69.5) (end 109 70.25) (width 0.254) (layer "B.Cu") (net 2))
 (segment (start 109 70.25) (end 109 80.25) (width 0.254) (layer "B.Cu") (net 2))
 (via (at 127.75 86.5) (size 0.508) (drill 0.254) (layers "F.Cu" "B.Cu") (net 2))
 (segment (start 109 80.25) (end 115.25 86.5) (width 0.254) (layer "B.Cu") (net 2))
 (segment (start 115.25 86.5) (end 127.75 86.5) (width 0.254) (layer "B.Cu") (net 2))
 (via (at 115.75 83.25) (size 0.508) (drill 0.254) (layers "F.Cu" "B.Cu") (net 1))
 (via (at 116.5 83.25) (size 0.508) (drill 0.254) (layers "F.Cu" "B.Cu") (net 1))
 (via (at 117.25 83.25) (size 0.508) (drill 0.254) (layers "F.Cu" "B.Cu") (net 1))
 (via (at 118 83.25) (size 0.508) (drill 0.254) (layers "F.Cu" "B.Cu") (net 1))
 (via (at 124.75 83.5) (size 0.508) (drill 0.254) (layers "F.Cu" "B.Cu") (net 1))
 (via (at 125.5 83.5) (size 0.508) (drill 0.254) (layers "F.Cu" "B.Cu") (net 1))
 (via (at 126.25 83.5) (size 0.508) (drill 0.254) (layers "F.Cu" "B.Cu") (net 1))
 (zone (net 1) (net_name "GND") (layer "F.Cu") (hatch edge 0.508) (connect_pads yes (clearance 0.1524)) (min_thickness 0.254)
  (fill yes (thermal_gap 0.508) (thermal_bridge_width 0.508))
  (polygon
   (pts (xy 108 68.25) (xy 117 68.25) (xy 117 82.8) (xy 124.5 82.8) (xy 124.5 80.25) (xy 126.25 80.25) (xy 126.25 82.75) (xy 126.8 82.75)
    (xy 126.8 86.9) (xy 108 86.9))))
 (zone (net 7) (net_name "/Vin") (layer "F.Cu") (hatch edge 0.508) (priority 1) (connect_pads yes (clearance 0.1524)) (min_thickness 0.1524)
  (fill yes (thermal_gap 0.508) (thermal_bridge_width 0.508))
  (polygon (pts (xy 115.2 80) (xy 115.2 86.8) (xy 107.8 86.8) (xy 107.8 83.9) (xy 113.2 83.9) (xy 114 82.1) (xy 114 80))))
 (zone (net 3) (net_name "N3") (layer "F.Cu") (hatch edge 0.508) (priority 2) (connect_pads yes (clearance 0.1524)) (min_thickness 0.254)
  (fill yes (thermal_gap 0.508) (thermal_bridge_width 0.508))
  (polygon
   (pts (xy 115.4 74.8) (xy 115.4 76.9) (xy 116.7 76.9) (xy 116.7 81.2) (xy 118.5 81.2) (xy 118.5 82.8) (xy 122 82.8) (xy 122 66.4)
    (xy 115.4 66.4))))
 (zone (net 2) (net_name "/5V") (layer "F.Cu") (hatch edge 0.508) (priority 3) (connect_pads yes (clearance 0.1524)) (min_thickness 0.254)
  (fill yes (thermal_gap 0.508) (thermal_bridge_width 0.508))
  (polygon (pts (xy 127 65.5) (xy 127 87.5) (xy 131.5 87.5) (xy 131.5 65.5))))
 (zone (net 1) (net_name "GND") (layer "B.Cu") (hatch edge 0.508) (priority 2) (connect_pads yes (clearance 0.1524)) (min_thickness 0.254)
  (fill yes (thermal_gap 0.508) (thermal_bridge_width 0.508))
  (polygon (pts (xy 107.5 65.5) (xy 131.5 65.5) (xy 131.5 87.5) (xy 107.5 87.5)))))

